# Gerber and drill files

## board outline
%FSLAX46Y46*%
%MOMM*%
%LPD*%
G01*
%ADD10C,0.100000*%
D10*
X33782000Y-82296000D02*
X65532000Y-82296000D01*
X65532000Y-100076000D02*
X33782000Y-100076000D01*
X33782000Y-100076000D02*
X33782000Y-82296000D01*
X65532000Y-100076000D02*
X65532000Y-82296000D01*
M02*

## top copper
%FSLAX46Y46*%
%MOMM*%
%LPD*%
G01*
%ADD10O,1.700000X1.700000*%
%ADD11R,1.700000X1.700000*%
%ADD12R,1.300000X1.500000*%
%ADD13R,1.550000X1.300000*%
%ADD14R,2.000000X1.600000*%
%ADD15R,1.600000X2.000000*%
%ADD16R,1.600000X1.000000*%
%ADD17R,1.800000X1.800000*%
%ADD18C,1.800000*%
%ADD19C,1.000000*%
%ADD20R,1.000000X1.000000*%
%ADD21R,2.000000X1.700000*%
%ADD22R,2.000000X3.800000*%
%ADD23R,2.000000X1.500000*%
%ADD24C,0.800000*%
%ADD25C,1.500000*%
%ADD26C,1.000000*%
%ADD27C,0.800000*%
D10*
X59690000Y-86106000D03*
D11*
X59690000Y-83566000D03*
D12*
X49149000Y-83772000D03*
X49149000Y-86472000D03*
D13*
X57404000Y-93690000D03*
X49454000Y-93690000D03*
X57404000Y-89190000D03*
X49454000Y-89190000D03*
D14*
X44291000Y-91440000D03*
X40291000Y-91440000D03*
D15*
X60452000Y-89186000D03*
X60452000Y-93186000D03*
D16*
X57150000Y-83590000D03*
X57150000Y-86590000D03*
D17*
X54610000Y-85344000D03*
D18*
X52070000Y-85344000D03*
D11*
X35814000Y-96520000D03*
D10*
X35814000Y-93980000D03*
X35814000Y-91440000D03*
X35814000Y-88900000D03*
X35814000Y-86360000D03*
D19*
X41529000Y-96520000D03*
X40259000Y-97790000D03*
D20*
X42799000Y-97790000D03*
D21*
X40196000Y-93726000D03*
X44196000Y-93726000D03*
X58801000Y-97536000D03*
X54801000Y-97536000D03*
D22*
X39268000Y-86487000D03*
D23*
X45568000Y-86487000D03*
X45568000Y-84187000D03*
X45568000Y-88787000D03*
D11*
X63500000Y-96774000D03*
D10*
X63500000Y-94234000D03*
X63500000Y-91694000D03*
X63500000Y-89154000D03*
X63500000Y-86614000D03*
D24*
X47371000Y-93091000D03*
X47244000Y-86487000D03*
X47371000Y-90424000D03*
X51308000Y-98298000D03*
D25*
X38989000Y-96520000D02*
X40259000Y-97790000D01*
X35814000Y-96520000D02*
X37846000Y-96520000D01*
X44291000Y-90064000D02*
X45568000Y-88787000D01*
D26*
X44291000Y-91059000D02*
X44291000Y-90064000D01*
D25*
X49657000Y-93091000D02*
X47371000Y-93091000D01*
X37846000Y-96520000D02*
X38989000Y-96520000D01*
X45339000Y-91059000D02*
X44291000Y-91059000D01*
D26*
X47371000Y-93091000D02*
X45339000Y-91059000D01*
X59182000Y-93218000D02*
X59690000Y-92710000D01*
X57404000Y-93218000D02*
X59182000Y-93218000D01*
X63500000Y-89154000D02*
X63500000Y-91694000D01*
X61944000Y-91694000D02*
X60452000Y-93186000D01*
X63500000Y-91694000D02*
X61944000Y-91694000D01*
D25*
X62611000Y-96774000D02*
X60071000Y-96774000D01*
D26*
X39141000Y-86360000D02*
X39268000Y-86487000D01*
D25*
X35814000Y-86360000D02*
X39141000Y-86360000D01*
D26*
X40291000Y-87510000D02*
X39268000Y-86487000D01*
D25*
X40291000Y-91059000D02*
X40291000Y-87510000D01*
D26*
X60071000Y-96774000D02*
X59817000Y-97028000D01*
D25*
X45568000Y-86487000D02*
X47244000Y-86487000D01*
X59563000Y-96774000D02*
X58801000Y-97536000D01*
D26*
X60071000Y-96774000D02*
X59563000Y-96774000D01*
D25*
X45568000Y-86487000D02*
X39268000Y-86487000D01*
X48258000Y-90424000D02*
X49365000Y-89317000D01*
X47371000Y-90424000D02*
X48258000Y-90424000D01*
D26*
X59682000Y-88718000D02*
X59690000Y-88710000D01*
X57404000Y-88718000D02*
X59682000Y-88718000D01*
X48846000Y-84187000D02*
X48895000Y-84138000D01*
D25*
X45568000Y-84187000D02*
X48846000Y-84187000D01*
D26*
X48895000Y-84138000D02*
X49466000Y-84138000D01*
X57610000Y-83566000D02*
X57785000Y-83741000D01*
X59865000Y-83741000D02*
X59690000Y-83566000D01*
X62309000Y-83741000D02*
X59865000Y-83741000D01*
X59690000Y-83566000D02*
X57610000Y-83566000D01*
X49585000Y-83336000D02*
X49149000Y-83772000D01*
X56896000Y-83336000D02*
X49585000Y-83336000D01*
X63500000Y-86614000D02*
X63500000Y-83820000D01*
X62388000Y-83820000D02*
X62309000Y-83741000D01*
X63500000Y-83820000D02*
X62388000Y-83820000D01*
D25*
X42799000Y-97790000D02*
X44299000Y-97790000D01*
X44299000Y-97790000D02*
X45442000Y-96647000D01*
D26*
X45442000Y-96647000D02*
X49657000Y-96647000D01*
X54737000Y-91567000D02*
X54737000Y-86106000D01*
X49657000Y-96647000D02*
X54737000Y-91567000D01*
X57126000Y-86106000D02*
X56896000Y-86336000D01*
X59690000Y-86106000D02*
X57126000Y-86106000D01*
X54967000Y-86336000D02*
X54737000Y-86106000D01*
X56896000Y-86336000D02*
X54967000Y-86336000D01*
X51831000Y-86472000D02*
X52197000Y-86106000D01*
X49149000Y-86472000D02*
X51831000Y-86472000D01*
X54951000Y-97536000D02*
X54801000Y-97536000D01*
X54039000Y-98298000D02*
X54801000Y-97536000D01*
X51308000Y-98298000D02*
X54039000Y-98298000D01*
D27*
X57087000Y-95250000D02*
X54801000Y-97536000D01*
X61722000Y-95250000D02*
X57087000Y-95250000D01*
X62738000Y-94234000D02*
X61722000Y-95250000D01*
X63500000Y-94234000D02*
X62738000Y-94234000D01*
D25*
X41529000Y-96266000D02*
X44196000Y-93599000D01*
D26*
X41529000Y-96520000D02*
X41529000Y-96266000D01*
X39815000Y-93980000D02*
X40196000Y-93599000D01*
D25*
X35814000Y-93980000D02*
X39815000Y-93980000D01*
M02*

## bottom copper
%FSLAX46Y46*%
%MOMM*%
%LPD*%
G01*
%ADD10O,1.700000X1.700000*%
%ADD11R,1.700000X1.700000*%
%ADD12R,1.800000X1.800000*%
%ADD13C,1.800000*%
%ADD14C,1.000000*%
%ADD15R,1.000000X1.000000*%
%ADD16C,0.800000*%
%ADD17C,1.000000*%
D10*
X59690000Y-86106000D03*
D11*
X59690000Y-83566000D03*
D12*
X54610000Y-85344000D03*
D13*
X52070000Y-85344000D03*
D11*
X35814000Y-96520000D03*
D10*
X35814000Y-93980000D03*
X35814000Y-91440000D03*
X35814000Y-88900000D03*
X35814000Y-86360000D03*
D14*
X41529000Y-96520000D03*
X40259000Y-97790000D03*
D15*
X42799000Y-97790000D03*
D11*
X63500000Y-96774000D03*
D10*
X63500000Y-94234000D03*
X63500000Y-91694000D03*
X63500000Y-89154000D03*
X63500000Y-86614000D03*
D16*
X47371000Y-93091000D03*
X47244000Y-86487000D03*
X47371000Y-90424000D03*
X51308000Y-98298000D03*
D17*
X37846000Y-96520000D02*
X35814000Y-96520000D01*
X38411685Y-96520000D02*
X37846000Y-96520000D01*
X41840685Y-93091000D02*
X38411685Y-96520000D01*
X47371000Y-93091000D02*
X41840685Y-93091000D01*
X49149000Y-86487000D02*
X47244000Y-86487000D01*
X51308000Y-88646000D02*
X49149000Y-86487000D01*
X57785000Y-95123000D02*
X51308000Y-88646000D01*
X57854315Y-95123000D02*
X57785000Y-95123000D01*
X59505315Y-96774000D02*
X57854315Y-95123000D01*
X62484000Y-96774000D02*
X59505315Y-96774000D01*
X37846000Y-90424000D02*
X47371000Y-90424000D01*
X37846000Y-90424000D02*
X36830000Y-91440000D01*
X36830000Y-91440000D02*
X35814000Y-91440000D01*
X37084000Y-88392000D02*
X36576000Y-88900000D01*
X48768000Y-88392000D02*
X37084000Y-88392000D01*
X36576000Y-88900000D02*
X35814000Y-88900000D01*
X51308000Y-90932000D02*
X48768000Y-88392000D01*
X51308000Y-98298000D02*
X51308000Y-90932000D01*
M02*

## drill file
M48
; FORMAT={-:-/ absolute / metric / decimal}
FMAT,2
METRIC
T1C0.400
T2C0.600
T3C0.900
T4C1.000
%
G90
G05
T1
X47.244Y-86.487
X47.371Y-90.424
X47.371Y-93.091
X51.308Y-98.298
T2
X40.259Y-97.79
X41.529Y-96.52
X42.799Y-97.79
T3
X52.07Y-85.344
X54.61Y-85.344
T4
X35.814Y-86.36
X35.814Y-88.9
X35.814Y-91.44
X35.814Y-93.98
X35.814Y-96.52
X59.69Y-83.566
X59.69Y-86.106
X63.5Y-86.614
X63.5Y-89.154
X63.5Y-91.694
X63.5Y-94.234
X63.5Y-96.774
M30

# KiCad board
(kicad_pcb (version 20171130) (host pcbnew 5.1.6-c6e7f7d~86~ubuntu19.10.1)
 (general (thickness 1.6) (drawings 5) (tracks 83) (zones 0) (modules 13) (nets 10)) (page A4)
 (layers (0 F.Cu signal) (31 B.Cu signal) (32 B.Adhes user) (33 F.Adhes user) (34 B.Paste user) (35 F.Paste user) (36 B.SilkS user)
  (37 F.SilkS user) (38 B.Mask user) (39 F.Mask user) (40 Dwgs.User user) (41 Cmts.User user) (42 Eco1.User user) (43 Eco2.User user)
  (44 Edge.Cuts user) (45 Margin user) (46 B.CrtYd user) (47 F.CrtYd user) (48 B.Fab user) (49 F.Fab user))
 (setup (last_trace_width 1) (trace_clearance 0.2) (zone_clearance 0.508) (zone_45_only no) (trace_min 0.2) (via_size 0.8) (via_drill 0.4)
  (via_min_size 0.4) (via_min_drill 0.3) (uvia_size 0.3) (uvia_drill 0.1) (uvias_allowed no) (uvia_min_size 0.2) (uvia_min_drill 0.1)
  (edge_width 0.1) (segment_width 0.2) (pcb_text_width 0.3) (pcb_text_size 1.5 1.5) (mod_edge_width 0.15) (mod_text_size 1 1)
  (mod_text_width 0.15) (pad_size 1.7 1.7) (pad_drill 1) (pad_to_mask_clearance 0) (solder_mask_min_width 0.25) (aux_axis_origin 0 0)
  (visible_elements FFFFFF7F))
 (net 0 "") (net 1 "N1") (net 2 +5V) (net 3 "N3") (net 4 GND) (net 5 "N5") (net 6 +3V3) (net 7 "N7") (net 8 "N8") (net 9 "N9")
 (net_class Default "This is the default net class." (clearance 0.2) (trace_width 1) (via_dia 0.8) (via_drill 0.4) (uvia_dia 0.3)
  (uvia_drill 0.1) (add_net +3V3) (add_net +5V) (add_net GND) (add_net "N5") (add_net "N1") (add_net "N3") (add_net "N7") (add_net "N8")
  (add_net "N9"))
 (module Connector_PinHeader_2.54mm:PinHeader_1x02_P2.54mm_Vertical (layer B.Cu) (at 59.69 83.566 180)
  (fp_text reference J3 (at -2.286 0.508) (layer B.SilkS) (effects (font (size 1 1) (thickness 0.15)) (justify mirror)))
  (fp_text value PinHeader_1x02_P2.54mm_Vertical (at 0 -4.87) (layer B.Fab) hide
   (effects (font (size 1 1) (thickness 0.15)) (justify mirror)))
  (pad 2 thru_hole oval (at 0 -2.54 180) (size 1.7 1.7) (drill 1) (layers *.Cu *.Mask) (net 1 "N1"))
  (pad 1 thru_hole rect (at 0 0 180) (size 1.7 1.7) (drill 1) (layers *.Cu *.Mask) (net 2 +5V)))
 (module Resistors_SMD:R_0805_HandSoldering (layer F.Cu) (at 49.149 85.122 90)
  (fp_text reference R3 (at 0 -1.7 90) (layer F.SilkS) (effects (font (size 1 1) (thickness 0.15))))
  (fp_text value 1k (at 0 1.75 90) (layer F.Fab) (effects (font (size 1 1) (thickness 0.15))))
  (pad 2 smd rect (at 1.35 0 90) (size 1.5 1.3) (layers F.Cu F.Paste F.Mask) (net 2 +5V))
  (pad 1 smd rect (at -1.35 0 90) (size 1.5 1.3) (layers F.Cu F.Paste F.Mask) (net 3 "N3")))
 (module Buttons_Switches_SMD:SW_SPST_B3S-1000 (layer F.Cu) (at 53.429 91.44)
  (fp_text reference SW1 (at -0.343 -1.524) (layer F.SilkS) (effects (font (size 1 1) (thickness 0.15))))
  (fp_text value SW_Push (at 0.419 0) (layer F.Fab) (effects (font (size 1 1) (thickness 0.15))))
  (pad 2 smd rect (at 3.975 2.25) (size 1.55 1.3) (layers F.Cu F.Paste F.Mask) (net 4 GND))
  (pad 2 smd rect (at -3.975 2.25) (size 1.55 1.3) (layers F.Cu F.Paste F.Mask) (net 4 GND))
  (pad 1 smd rect (at 3.975 -2.25) (size 1.55 1.3) (layers F.Cu F.Paste F.Mask) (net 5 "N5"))
  (pad 1 smd rect (at -3.975 -2.25) (size 1.55 1.3) (layers F.Cu F.Paste F.Mask) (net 5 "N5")))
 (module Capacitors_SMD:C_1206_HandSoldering (layer F.Cu) (at 42.291 91.44)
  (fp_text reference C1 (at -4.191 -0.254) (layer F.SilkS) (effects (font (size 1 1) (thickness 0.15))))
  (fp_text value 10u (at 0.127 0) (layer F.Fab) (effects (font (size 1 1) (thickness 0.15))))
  (pad 2 smd rect (at 2 0) (size 2 1.6) (layers F.Cu F.Paste F.Mask) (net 4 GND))
  (pad 1 smd rect (at -2 0) (size 2 1.6) (layers F.Cu F.Paste F.Mask) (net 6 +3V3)))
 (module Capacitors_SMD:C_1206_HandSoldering (layer F.Cu) (at 60.452 91.186 270)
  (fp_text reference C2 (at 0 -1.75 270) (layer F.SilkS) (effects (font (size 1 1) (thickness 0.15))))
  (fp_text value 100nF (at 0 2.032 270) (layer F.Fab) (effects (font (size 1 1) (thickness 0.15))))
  (pad 1 smd rect (at -2 0 270) (size 2 1.6) (layers F.Cu F.Paste F.Mask) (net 5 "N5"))
  (pad 2 smd rect (at 2 0 270) (size 2 1.6) (layers F.Cu F.Paste F.Mask) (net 4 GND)))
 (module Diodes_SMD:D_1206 (layer F.Cu) (at 57.15 85.09 270)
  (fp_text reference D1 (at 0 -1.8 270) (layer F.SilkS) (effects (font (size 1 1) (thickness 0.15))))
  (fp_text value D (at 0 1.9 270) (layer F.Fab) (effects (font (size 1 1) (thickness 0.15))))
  (pad 1 smd rect (at -1.5 0 270) (size 1 1.6) (layers F.Cu F.Paste F.Mask) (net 2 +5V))
  (pad 2 smd rect (at 1.5 0 270) (size 1 1.6) (layers F.Cu F.Paste F.Mask) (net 1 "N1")))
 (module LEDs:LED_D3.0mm (layer F.Cu) (at 54.61 85.344 180)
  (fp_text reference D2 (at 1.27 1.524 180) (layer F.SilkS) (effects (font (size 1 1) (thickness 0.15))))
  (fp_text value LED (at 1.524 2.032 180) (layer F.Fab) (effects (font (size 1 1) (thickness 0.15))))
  (pad 1 thru_hole rect (at 0 0 180) (size 1.8 1.8) (drill 0.9) (layers *.Cu *.Mask) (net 1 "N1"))
  (pad 2 thru_hole circle (at 2.54 0 180) (size 1.8 1.8) (drill 0.9) (layers *.Cu *.Mask) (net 3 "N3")))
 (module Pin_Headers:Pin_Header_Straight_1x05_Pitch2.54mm (layer B.Cu) (at 35.814 96.52)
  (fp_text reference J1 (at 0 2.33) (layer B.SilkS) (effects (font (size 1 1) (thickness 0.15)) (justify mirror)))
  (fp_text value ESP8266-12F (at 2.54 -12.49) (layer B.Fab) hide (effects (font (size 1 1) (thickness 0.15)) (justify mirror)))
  (pad 1 thru_hole rect (at 0 0) (size 1.7 1.7) (drill 1) (layers *.Cu *.Mask) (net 4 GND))
  (pad 2 thru_hole oval (at 0 -2.54) (size 1.7 1.7) (drill 1) (layers *.Cu *.Mask) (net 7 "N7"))
  (pad 3 thru_hole oval (at 0 -5.08) (size 1.7 1.7) (drill 1) (layers *.Cu *.Mask) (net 5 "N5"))
  (pad 4 thru_hole oval (at 0 -7.62) (size 1.7 1.7) (drill 1) (layers *.Cu *.Mask) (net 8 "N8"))
  (pad 5 thru_hole oval (at 0 -10.16) (size 1.7 1.7) (drill 1) (layers *.Cu *.Mask) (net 6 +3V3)))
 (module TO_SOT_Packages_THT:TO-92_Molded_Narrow (layer B.Cu) (at 42.799 97.79 180)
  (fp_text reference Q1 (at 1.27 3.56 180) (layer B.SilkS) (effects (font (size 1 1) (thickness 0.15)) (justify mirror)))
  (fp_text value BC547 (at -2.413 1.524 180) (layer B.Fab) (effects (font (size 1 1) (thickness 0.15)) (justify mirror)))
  (pad 2 thru_hole circle (at 1.27 1.27 90) (size 1 1) (drill 0.6) (layers *.Cu *.Mask) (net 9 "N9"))
  (pad 3 thru_hole circle (at 2.54 0 90) (size 1 1) (drill 0.6) (layers *.Cu *.Mask) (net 4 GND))
  (pad 1 thru_hole rect (at 0 0 90) (size 1 1) (drill 0.6) (layers *.Cu *.Mask) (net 1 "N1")))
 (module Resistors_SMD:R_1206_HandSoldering (layer F.Cu) (at 42.196 93.726)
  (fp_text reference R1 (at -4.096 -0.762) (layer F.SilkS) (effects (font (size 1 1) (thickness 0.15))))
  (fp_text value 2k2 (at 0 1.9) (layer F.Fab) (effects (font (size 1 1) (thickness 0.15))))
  (pad 1 smd rect (at -2 0) (size 2 1.7) (layers F.Cu F.Paste F.Mask) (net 7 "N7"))
  (pad 2 smd rect (at 2 0) (size 2 1.7) (layers F.Cu F.Paste F.Mask) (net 9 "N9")))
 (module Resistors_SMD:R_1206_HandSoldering (layer F.Cu) (at 56.801 97.536)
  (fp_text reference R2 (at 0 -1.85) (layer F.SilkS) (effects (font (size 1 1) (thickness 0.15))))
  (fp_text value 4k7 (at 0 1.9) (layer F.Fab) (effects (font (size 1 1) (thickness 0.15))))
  (pad 2 smd rect (at 2 0) (size 2 1.7) (layers F.Cu F.Paste F.Mask) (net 6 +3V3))
  (pad 1 smd rect (at -2 0) (size 2 1.7) (layers F.Cu F.Paste F.Mask) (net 8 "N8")))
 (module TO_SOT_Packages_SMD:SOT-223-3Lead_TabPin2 (layer F.Cu) (at 42.418 86.487 180)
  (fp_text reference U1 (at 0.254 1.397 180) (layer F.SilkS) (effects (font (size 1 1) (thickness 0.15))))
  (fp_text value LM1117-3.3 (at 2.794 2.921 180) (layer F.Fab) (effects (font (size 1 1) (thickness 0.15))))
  (pad 2 smd rect (at 3.15 0 180) (size 2 3.8) (layers F.Cu F.Paste F.Mask) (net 6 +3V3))
  (pad 2 smd rect (at -3.15 0 180) (size 2 1.5) (layers F.Cu F.Paste F.Mask) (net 6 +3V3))
  (pad 3 smd rect (at -3.15 2.3 180) (size 2 1.5) (layers F.Cu F.Paste F.Mask) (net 2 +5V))
  (pad 1 smd rect (at -3.15 -2.3 180) (size 2 1.5) (layers F.Cu F.Paste F.Mask) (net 4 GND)))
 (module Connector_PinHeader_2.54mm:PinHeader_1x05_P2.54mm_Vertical (layer B.Cu) (at 63.5 96.774)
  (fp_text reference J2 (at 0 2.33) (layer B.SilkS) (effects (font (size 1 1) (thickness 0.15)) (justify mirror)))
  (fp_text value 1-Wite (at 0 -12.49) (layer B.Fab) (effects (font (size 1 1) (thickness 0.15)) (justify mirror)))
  (pad 1 thru_hole rect (at 0 0) (size 1.7 1.7) (drill 1) (layers *.Cu *.Mask) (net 6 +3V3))
  (pad 2 thru_hole oval (at 0 -2.54) (size 1.7 1.7) (drill 1) (layers *.Cu *.Mask) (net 8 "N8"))
  (pad 3 thru_hole oval (at 0 -5.08) (size 1.7 1.7) (drill 1) (layers *.Cu *.Mask) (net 4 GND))
  (pad 4 thru_hole oval (at 0 -7.62) (size 1.7 1.7) (drill 1) (layers *.Cu *.Mask) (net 4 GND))
  (pad 5 thru_hole oval (at 0 -10.16) (size 1.7 1.7) (drill 1) (layers *.Cu *.Mask) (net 2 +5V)))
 (gr_line (start 33.782 82.296) (end 65.532 82.296) (layer Edge.Cuts) (width 0.1))
 (gr_line (start 65.532 100.076) (end 33.782 100.076) (layer Edge.Cuts) (width 0.1))
 (gr_line (start 33.782 100.076) (end 33.782 82.296) (layer Edge.Cuts) (width 0.1))
 (gr_line (start 65.532 100.076) (end 65.532 82.296) (layer Edge.Cuts) (width 0.1))
 (segment (start 38.989 96.52) (end 40.259 97.79) (width 1.5) (layer F.Cu) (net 4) (status 20))
 (segment (start 35.814 96.52) (end 37.846 96.52) (width 1.5) (layer F.Cu) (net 4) (status 10))
 (segment (start 44.291 90.064) (end 45.568 88.787) (width 1.5) (layer F.Cu) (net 4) (status 20))
 (segment (start 44.291 91.059) (end 44.291 90.064) (width 1) (layer F.Cu) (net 4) (status 10))
 (segment (start 49.657 93.091) (end 47.371 93.091) (width 1.5) (layer F.Cu) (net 4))
 (segment (start 37.846 96.52) (end 38.989 96.52) (width 1.5) (layer F.Cu) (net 4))
 (via (at 47.371 93.091) (size 0.8) (drill 0.4) (layers F.Cu B.Cu) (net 4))
 (segment (start 45.339 91.059) (end 44.291 91.059) (width 1.5) (layer F.Cu) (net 4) (status 20))
 (segment (start 47.371 93.091) (end 45.339 91.059) (width 1) (layer F.Cu) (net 4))
 (segment (start 37.846 96.52) (end 35.814 96.52) (width 1) (layer B.Cu) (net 4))
 (segment (start 38.411685 96.52) (end 37.846 96.52) (width 1) (layer B.Cu) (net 4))
 (segment (start 41.840685 93.091) (end 38.411685 96.52) (width 1) (layer B.Cu) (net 4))
 (segment (start 47.371 93.091) (end 41.840685 93.091) (width 1) (layer B.Cu) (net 4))
 (segment (start 59.182 93.218) (end 59.69 92.71) (width 1) (layer F.Cu) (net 4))
 (segment (start 57.404 93.218) (end 59.182 93.218) (width 1) (layer F.Cu) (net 4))
 (segment (start 63.5 89.154) (end 63.5 91.694) (width 1) (layer F.Cu) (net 4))
 (segment (start 61.944 91.694) (end 60.452 93.186) (width 1) (layer F.Cu) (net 4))
 (segment (start 63.5 91.694) (end 61.944 91.694) (width 1) (layer F.Cu) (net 4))
 (segment (start 62.611 96.774) (end 60.071 96.774) (width 1.5) (layer F.Cu) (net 6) (status 10))
 (segment (start 39.141 86.36) (end 39.268 86.487) (width 1) (layer F.Cu) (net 6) (status 30))
 (segment (start 35.814 86.36) (end 39.141 86.36) (width 1.5) (layer F.Cu) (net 6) (status 30))
 (segment (start 40.291 87.51) (end 39.268 86.487) (width 1) (layer F.Cu) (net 6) (status 20))
 (segment (start 40.291 91.059) (end 40.291 87.51) (width 1.5) (layer F.Cu) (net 6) (status 10))
 (segment (start 60.071 96.774) (end 59.817 97.028) (width 1) (layer F.Cu) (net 6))
 (segment (start 45.568 86.487) (end 47.244 86.487) (width 1.5) (layer F.Cu) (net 6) (status 10))
 (via (at 47.244 86.487) (size 0.8) (drill 0.4) (layers F.Cu B.Cu) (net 6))
 (segment (start 49.149 86.487) (end 47.244 86.487) (width 1) (layer B.Cu) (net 6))
 (segment (start 51.308 88.646) (end 49.149 86.487) (width 1) (layer B.Cu) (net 6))
 (segment (start 59.563 96.774) (end 58.801 97.536) (width 1.5) (layer F.Cu) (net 6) (status 30))
 (segment (start 60.071 96.774) (end 59.563 96.774) (width 1) (layer F.Cu) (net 6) (status 20))
 (segment (start 45.568 86.487) (end 39.268 86.487) (width 1.5) (layer F.Cu) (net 6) (status 30))
 (segment (start 57.785 95.123) (end 51.308 88.646) (width 1) (layer B.Cu) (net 6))
 (segment (start 57.854315 95.123) (end 57.785 95.123) (width 1) (layer B.Cu) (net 6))
 (segment (start 59.505315 96.774) (end 57.854315 95.123) (width 1) (layer B.Cu) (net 6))
 (segment (start 62.484 96.774) (end 59.505315 96.774) (width 1) (layer B.Cu) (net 6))
 (via (at 47.371 90.424) (size 0.8) (drill 0.4) (layers F.Cu B.Cu) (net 5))
 (segment (start 37.846 90.424) (end 47.371 90.424) (width 1) (layer B.Cu) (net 5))
 (segment (start 48.258 90.424) (end 49.365 89.317) (width 1.5) (layer F.Cu) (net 5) (status 20))
 (segment (start 47.371 90.424) (end 48.258 90.424) (width 1.5) (layer F.Cu) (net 5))
 (segment (start 37.846 90.424) (end 36.83 91.44) (width 1) (layer B.Cu) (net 5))
 (segment (start 36.83 91.44) (end 35.814 91.44) (width 1) (layer B.Cu) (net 5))
 (segment (start 59.682 88.718) (end 59.69 88.71) (width 1) (layer F.Cu) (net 5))
 (segment (start 57.404 88.718) (end 59.682 88.718) (width 1) (layer F.Cu) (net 5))
 (segment (start 48.846 84.187) (end 48.895 84.138) (width 1) (layer F.Cu) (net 2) (status 30))
 (segment (start 45.568 84.187) (end 48.846 84.187) (width 1.5) (layer F.Cu) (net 2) (status 30))
 (segment (start 48.895 84.138) (end 49.466 84.138) (width 1) (layer F.Cu) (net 2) (status 30))
 (segment (start 57.61 83.566) (end 57.785 83.741) (width 1) (layer F.Cu) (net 2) (status 30))
 (segment (start 59.865 83.741) (end 59.69 83.566) (width 1) (layer F.Cu) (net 2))
 (segment (start 62.309 83.741) (end 59.865 83.741) (width 1) (layer F.Cu) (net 2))
 (segment (start 59.69 83.566) (end 57.61 83.566) (width 1) (layer F.Cu) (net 2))
 (segment (start 49.585 83.336) (end 49.149 83.772) (width 1) (layer F.Cu) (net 2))
 (segment (start 56.896 83.336) (end 49.585 83.336) (width 1) (layer F.Cu) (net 2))
 (segment (start 63.5 86.614) (end 63.5 83.82) (width 1) (layer F.Cu) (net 2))
 (segment (start 62.388 83.82) (end 62.309 83.741) (width 1) (layer F.Cu) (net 2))
 (segment (start 63.5 83.82) (end 62.388 83.82) (width 1) (layer F.Cu) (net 2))
 (segment (start 42.799 97.79) (end 44.299 97.79) (width 1.5) (layer F.Cu) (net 1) (status 10))
 (segment (start 44.299 97.79) (end 45.442 96.647) (width 1.5) (layer F.Cu) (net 1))
 (segment (start 45.442 96.647) (end 49.657 96.647) (width 1) (layer F.Cu) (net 1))
 (segment (start 54.737 91.567) (end 54.737 86.106) (width 1) (layer F.Cu) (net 1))
 (segment (start 49.657 96.647) (end 54.737 91.567) (width 1) (layer F.Cu) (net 1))
 (segment (start 57.126 86.106) (end 56.896 86.336) (width 1) (layer F.Cu) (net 1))
 (segment (start 59.69 86.106) (end 57.126 86.106) (width 1) (layer F.Cu) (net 1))
 (segment (start 54.967 86.336) (end 54.737 86.106) (width 1) (layer F.Cu) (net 1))
 (segment (start 56.896 86.336) (end 54.967 86.336) (width 1) (layer F.Cu) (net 1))
 (segment (start 51.831 86.472) (end 52.197 86.106) (width 1) (layer F.Cu) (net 3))
 (segment (start 49.149 86.472) (end 51.831 86.472) (width 1) (layer F.Cu) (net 3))
 (segment (start 54.951 97.536) (end 54.801 97.536) (width 1) (layer F.Cu) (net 8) (status 30))
 (via (at 51.308 98.298) (size 0.8) (drill 0.4) (layers F.Cu B.Cu) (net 8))
 (segment (start 54.039 98.298) (end 54.801 97.536) (width 1) (layer F.Cu) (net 8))
 (segment (start 51.308 98.298) (end 54.039 98.298) (width 1) (layer F.Cu) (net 8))
 (segment (start 37.084 88.392) (end 36.576 88.9) (width 1) (layer B.Cu) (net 8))
 (segment (start 48.768 88.392) (end 37.084 88.392) (width 1) (layer B.Cu) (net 8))
 (segment (start 36.576 88.9) (end 35.814 88.9) (width 1) (layer B.Cu) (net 8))
 (segment (start 51.308 90.932) (end 48.768 88.392) (width 1) (layer B.Cu) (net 8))
 (segment (start 51.308 98.298) (end 51.308 90.932) (width 1) (layer B.Cu) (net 8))
 (segment (start 57.087 95.25) (end 54.801 97.536) (width 0.8) (layer F.Cu) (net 8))
 (segment (start 61.722 95.25) (end 57.087 95.25) (width 0.8) (layer F.Cu) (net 8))
 (segment (start 62.738 94.234) (end 61.722 95.25) (width 0.8) (layer F.Cu) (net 8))
 (segment (start 63.5 94.234) (end 62.738 94.234) (width 0.8) (layer F.Cu) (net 8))
 (segment (start 41.529 96.266) (end 44.196 93.599) (width 1.5) (layer F.Cu) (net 9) (status 30))
 (segment (start 41.529 96.52) (end 41.529 96.266) (width 1) (layer F.Cu) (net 9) (status 30))
 (segment (start 39.815 93.98) (end 40.196 93.599) (width 1) (layer F.Cu) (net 7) (status 30))
 (segment (start 35.814 93.98) (end 39.815 93.98) (width 1.5) (layer F.Cu) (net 7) (status 30)))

